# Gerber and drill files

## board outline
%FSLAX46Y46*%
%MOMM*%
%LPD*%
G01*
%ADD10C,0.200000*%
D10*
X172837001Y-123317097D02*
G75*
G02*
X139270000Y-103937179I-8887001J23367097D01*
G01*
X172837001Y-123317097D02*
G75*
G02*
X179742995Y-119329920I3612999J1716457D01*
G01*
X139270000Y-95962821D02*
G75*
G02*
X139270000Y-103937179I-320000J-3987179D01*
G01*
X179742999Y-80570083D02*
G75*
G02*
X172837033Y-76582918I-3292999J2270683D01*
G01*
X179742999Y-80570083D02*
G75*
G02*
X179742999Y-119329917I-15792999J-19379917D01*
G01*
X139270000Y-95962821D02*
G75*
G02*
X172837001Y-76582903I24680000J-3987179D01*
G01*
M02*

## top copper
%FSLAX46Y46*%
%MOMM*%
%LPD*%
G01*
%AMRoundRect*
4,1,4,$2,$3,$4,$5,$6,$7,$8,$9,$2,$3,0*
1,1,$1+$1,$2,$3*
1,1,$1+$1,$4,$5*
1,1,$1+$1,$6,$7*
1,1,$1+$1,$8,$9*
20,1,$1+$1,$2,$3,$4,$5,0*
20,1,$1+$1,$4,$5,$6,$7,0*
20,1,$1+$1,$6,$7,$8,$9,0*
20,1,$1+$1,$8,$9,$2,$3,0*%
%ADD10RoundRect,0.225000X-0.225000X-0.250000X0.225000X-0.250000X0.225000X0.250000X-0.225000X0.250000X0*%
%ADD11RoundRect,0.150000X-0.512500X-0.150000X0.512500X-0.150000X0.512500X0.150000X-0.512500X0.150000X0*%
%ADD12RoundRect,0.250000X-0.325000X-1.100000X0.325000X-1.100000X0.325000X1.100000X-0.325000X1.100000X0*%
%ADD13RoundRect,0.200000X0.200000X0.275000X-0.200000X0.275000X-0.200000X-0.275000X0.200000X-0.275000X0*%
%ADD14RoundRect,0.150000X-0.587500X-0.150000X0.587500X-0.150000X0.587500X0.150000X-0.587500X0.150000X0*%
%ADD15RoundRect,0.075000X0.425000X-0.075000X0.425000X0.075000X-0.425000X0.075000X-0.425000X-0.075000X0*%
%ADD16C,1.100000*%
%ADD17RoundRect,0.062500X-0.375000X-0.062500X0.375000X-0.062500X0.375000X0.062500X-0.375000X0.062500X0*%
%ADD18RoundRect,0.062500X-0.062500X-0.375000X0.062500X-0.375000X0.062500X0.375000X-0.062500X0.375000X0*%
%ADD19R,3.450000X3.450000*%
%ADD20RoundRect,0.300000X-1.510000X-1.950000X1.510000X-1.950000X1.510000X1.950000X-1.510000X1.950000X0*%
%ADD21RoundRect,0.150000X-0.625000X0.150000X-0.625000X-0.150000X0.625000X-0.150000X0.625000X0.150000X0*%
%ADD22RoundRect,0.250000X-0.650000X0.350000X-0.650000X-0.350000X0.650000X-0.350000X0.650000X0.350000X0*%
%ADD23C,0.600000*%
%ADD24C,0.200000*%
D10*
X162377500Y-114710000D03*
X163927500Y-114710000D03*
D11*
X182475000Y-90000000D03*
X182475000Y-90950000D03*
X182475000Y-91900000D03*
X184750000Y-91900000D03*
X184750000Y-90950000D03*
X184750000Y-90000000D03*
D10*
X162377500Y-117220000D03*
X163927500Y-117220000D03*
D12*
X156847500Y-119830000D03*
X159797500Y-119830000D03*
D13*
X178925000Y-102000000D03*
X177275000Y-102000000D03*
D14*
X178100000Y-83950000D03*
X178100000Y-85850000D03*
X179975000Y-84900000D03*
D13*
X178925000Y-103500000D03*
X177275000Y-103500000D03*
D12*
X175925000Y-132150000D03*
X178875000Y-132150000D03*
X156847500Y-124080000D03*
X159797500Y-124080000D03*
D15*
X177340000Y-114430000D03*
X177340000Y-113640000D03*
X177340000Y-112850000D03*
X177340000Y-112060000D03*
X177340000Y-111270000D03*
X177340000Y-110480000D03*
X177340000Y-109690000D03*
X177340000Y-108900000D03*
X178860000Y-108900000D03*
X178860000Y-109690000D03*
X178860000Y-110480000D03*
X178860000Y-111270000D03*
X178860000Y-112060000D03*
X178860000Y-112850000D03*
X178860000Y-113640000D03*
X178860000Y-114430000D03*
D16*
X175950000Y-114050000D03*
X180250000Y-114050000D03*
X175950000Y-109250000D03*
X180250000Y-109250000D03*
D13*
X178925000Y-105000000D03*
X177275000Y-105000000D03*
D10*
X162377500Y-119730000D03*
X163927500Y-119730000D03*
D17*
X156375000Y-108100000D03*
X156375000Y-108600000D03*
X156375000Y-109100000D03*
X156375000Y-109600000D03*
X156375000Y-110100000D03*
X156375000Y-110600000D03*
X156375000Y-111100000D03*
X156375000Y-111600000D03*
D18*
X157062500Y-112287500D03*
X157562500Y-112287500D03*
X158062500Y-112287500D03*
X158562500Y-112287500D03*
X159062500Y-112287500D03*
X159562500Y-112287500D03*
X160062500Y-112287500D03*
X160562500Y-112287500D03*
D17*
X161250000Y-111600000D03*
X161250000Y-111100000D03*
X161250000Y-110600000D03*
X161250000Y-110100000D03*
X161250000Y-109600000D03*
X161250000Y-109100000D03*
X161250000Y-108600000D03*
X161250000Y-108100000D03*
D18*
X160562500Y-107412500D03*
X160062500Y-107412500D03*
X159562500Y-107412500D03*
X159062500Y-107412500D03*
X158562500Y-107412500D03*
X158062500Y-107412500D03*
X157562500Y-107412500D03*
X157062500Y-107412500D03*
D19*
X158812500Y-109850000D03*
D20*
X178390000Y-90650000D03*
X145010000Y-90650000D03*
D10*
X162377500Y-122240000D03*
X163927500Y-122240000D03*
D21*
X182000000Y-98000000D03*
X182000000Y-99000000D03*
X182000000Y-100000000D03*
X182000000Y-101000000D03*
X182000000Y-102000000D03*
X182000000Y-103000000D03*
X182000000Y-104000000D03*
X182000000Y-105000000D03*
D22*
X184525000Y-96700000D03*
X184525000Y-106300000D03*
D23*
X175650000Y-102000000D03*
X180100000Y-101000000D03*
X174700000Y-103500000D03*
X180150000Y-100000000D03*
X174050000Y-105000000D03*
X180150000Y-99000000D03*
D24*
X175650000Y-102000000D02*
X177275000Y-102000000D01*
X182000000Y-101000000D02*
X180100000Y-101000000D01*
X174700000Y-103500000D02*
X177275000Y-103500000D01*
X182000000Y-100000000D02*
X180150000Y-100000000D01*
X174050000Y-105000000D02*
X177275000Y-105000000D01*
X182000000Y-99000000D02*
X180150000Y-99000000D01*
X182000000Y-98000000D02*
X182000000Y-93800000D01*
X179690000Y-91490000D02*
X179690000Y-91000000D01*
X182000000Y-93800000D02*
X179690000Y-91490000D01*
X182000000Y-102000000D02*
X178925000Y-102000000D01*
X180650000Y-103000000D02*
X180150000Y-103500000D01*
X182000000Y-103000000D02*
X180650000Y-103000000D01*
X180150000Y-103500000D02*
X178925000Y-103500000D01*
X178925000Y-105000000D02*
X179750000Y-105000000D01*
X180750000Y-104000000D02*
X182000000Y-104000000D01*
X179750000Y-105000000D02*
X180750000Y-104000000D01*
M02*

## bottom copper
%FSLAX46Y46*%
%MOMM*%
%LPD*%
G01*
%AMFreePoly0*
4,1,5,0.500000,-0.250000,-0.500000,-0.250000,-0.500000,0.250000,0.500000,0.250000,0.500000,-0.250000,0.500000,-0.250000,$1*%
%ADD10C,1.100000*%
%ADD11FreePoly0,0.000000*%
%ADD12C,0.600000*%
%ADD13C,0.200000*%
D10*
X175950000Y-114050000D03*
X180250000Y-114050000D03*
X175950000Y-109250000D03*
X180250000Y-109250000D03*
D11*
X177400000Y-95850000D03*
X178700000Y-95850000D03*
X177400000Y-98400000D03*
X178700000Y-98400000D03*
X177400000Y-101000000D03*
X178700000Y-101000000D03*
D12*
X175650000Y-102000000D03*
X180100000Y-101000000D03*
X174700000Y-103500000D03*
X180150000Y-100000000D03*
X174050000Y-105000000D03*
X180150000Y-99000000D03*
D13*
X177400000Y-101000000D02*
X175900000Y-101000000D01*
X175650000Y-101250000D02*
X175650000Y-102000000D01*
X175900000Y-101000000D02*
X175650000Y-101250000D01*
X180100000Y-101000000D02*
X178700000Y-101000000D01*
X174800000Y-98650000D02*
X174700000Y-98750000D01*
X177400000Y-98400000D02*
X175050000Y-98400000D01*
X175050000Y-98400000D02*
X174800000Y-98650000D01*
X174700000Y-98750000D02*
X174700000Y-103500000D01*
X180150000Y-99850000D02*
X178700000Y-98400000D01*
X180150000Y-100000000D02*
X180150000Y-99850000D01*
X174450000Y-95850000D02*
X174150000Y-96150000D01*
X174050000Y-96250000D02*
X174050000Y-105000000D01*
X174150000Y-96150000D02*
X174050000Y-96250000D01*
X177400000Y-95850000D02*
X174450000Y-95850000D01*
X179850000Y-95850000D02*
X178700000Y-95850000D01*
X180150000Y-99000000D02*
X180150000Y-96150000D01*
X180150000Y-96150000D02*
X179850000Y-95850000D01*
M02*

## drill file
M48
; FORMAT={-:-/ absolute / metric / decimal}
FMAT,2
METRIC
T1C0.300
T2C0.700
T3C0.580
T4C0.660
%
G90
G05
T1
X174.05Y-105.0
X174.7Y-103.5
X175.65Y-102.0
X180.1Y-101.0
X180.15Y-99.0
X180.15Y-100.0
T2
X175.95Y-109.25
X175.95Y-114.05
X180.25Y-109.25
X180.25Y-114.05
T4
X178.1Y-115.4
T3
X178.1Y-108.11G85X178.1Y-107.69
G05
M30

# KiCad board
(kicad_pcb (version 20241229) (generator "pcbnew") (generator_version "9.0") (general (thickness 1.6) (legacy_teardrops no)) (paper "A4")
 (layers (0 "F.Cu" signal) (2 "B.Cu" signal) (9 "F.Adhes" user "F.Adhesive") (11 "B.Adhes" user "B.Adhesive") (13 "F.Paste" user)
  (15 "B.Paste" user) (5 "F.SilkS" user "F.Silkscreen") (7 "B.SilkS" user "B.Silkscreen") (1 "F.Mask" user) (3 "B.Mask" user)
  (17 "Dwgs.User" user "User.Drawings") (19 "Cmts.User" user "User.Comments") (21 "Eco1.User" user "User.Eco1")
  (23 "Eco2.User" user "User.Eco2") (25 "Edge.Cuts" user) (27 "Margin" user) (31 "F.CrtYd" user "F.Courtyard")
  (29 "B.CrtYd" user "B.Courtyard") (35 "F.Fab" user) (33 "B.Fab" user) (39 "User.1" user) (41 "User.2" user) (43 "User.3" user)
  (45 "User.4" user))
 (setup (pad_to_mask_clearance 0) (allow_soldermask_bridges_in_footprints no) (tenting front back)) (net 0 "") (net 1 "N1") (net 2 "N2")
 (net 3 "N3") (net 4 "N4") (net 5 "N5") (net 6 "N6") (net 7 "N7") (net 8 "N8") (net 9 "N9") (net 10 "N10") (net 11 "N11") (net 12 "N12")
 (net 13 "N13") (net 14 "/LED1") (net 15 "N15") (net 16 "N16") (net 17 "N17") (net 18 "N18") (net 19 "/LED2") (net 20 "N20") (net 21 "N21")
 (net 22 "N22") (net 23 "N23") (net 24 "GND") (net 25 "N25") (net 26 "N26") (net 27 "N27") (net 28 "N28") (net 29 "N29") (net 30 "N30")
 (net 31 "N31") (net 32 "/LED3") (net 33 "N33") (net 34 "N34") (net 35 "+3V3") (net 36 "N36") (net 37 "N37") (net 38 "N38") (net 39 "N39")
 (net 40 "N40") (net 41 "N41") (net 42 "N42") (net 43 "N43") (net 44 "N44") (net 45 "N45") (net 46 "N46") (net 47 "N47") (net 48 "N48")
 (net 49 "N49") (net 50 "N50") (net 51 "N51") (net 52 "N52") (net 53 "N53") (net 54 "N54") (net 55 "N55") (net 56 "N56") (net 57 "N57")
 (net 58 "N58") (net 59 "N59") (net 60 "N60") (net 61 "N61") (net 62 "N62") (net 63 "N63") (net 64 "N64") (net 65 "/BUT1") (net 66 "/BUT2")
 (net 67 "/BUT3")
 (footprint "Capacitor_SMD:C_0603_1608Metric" (layer "F.Cu") (at 163.1525 114.71)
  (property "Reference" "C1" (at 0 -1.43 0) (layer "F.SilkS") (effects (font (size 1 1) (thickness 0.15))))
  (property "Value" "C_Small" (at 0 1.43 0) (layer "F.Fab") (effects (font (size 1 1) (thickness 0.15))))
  (pad "1" smd roundrect (at -0.775 0) (size 0.9 0.95) (layers "F.Cu" "F.Mask" "F.Paste") (roundrect_rratio 0.25) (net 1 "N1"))
  (pad "2" smd roundrect (at 0.775 0) (size 0.9 0.95) (layers "F.Cu" "F.Mask" "F.Paste") (roundrect_rratio 0.25) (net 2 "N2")))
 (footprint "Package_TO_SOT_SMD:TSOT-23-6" (layer "F.Cu") (at 183.6125 90.95)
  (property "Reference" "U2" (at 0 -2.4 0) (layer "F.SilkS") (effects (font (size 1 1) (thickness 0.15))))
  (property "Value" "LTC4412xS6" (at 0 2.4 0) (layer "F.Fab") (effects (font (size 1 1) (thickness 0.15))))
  (pad "1" smd roundrect (at -1.1375 -0.95) (size 1.325 0.6) (layers "F.Cu" "F.Mask" "F.Paste") (roundrect_rratio 0.25) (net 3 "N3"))
  (pad "2" smd roundrect (at -1.1375 0) (size 1.325 0.6) (layers "F.Cu" "F.Mask" "F.Paste") (roundrect_rratio 0.25) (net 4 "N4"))
  (pad "3" smd roundrect (at -1.1375 0.95) (size 1.325 0.6) (layers "F.Cu" "F.Mask" "F.Paste") (roundrect_rratio 0.25) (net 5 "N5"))
  (pad "4" smd roundrect (at 1.1375 0.95) (size 1.325 0.6) (layers "F.Cu" "F.Mask" "F.Paste") (roundrect_rratio 0.25) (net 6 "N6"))
  (pad "5" smd roundrect (at 1.1375 0) (size 1.325 0.6) (layers "F.Cu" "F.Mask" "F.Paste") (roundrect_rratio 0.25) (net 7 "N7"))
  (pad "6" smd roundrect (at 1.1375 -0.95) (size 1.325 0.6) (layers "F.Cu" "F.Mask" "F.Paste") (roundrect_rratio 0.25) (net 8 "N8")))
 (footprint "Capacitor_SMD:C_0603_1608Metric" (layer "F.Cu") (at 163.1525 117.22)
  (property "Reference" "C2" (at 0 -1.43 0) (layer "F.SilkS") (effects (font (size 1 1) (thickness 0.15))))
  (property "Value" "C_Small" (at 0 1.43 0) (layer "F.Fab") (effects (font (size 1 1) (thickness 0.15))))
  (pad "1" smd roundrect (at -0.775 0) (size 0.9 0.95) (layers "F.Cu" "F.Mask" "F.Paste") (roundrect_rratio 0.25) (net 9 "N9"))
  (pad "2" smd roundrect (at 0.775 0) (size 0.9 0.95) (layers "F.Cu" "F.Mask" "F.Paste") (roundrect_rratio 0.25) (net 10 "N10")))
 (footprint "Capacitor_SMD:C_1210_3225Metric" (layer "F.Cu") (at 158.3225 119.83)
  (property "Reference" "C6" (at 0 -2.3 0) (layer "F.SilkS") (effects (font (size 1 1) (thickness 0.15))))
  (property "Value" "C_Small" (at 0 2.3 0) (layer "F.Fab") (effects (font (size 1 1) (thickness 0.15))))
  (pad "1" smd roundrect (at -1.475 0) (size 1.15 2.7) (layers "F.Cu" "F.Mask" "F.Paste") (roundrect_rratio 0.217391) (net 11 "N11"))
  (pad "2" smd roundrect (at 1.475 0) (size 1.15 2.7) (layers "F.Cu" "F.Mask" "F.Paste") (roundrect_rratio 0.217391) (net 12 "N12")))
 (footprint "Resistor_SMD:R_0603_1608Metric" (layer "F.Cu") (at 178.1 102 180)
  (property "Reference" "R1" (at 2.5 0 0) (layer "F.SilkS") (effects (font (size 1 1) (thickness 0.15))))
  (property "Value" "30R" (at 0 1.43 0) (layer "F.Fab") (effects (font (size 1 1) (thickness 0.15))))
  (pad "1" smd roundrect (at -0.825 0 180) (size 0.8 0.95) (layers "F.Cu" "F.Mask" "F.Paste") (roundrect_rratio 0.25) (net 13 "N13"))
  (pad "2" smd roundrect (at 0.825 0 180) (size 0.8 0.95) (layers "F.Cu" "F.Mask" "F.Paste") (roundrect_rratio 0.25) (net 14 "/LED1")))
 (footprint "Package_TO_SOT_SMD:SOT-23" (layer "F.Cu") (at 179.0375 84.9)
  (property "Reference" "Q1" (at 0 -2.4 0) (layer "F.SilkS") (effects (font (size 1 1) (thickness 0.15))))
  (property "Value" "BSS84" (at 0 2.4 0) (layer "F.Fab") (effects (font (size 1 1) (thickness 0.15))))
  (pad "1" smd roundrect (at -0.9375 -0.95) (size 1.475 0.6) (layers "F.Cu" "F.Mask" "F.Paste") (roundrect_rratio 0.25) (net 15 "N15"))
  (pad "2" smd roundrect (at -0.9375 0.95) (size 1.475 0.6) (layers "F.Cu" "F.Mask" "F.Paste") (roundrect_rratio 0.25) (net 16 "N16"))
  (pad "3" smd roundrect (at 0.9375 0) (size 1.475 0.6) (layers "F.Cu" "F.Mask" "F.Paste") (roundrect_rratio 0.25) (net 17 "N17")))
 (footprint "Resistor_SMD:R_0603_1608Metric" (layer "F.Cu") (at 178.1 103.5 180)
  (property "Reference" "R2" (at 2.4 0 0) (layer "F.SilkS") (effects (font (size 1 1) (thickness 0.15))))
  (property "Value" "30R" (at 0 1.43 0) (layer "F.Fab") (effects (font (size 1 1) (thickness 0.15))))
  (pad "1" smd roundrect (at -0.825 0 180) (size 0.8 0.95) (layers "F.Cu" "F.Mask" "F.Paste") (roundrect_rratio 0.25) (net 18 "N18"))
  (pad "2" smd roundrect (at 0.825 0 180) (size 0.8 0.95) (layers "F.Cu" "F.Mask" "F.Paste") (roundrect_rratio 0.25) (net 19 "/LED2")))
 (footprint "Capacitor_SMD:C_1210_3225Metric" (layer "F.Cu") (at 177.4 132.15)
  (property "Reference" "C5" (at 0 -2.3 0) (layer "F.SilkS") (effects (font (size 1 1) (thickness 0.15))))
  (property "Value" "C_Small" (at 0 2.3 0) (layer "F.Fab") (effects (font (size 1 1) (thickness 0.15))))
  (pad "1" smd roundrect (at -1.475 0) (size 1.15 2.7) (layers "F.Cu" "F.Mask" "F.Paste") (roundrect_rratio 0.217391) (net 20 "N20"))
  (pad "2" smd roundrect (at 1.475 0) (size 1.15 2.7) (layers "F.Cu" "F.Mask" "F.Paste") (roundrect_rratio 0.217391) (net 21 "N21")))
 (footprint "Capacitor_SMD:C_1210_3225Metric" (layer "F.Cu") (at 158.3225 124.08)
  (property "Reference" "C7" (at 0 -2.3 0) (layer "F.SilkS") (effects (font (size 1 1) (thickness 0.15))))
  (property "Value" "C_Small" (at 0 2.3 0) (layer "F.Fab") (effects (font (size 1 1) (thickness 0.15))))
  (pad "1" smd roundrect (at -1.475 0) (size 1.15 2.7) (layers "F.Cu" "F.Mask" "F.Paste") (roundrect_rratio 0.217391) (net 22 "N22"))
  (pad "2" smd roundrect (at 1.475 0) (size 1.15 2.7) (layers "F.Cu" "F.Mask" "F.Paste") (roundrect_rratio 0.217391) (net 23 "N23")))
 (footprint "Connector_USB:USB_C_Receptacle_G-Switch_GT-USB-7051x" (layer "F.Cu") (at 178.1 111.65 90)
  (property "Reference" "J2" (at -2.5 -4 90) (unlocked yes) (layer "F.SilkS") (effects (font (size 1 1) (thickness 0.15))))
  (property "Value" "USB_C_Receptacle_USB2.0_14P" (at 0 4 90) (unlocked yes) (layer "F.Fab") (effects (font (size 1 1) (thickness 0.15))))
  (pad "" np_thru_hole circle (at -3.75 0 90) (size 0.66 0.66) (drill 0.66) (layers "*.Cu" "*.Mask"))
  (pad "" np_thru_hole oval (at 3.75 0 90) (size 1 0.58) (drill oval 1 0.58) (layers "*.Cu" "*.Mask"))
  (pad "A1" smd roundrect (at -2.78 -0.76 90) (size 0.3 1) (layers "F.Cu" "F.Mask" "F.Paste") (roundrect_rratio 0.25) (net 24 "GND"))
  (pad "A4" smd roundrect (at -1.99 -0.76 90) (size 0.3 1) (layers "F.Cu" "F.Mask" "F.Paste") (roundrect_rratio 0.25) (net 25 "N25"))
  (pad "A5" smd roundrect (at -1.2 -0.76 90) (size 0.3 1) (layers "F.Cu" "F.Mask" "F.Paste") (roundrect_rratio 0.25) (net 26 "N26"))
  (pad "A6" smd roundrect (at -0.41 -0.76 90) (size 0.3 1) (layers "F.Cu" "F.Mask" "F.Paste") (roundrect_rratio 0.25) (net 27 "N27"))
  (pad "A7" smd roundrect (at 0.38 -0.76 90) (size 0.3 1) (layers "F.Cu" "F.Mask" "F.Paste") (roundrect_rratio 0.25) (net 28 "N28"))
  (pad "A8" smd roundrect (at 1.17 -0.76 90) (size 0.3 1) (layers "F.Cu" "F.Mask" "F.Paste") (roundrect_rratio 0.25))
  (pad "A9" smd roundrect (at 1.96 -0.76 90) (size 0.3 1) (layers "F.Cu" "F.Mask" "F.Paste") (roundrect_rratio 0.25) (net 25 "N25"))
  (pad "A12" smd roundrect (at 2.75 -0.76 90) (size 0.3 1) (layers "F.Cu" "F.Mask" "F.Paste") (roundrect_rratio 0.25) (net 24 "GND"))
  (pad "B1" smd roundrect (at 2.75 0.76 90) (size 0.3 1) (layers "F.Cu" "F.Mask" "F.Paste") (roundrect_rratio 0.25) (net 24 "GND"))
  (pad "B4" smd roundrect (at 1.96 0.76 90) (size 0.3 1) (layers "F.Cu" "F.Mask" "F.Paste") (roundrect_rratio 0.25) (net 25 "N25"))
  (pad "B5" smd roundrect (at 1.17 0.76 90) (size 0.3 1) (layers "F.Cu" "F.Mask" "F.Paste") (roundrect_rratio 0.25) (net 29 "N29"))
  (pad "B6" smd roundrect (at 0.38 0.76 90) (size 0.3 1) (layers "F.Cu" "F.Mask" "F.Paste") (roundrect_rratio 0.25) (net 27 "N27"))
  (pad "B7" smd roundrect (at -0.41 0.76 90) (size 0.3 1) (layers "F.Cu" "F.Mask" "F.Paste") (roundrect_rratio 0.25) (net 28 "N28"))
  (pad "B8" smd roundrect (at -1.2 0.76 90) (size 0.3 1) (layers "F.Cu" "F.Mask" "F.Paste") (roundrect_rratio 0.25))
  (pad "B9" smd roundrect (at -1.99 0.76 90) (size 0.3 1) (layers "F.Cu" "F.Mask" "F.Paste") (roundrect_rratio 0.25) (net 25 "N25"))
  (pad "B12" smd roundrect (at -2.78 0.76 90) (size 0.3 1) (layers "F.Cu" "F.Mask" "F.Paste") (roundrect_rratio 0.25) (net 24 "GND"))
  (pad "S1" thru_hole circle (at -2.4 -2.15 90) (size 1.1 1.1) (drill 0.7) (layers "*.Cu" "*.Mask" "F.Paste") (remove_unused_layers no)
   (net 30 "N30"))
  (pad "S1" thru_hole circle (at -2.4 2.15 90) (size 1.1 1.1) (drill 0.7) (layers "*.Cu" "*.Mask" "F.Paste") (remove_unused_layers no)
   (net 30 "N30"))
  (pad "S1" thru_hole circle (at 2.4 -2.15 90) (size 1.1 1.1) (drill 0.7) (layers "*.Cu" "*.Mask" "F.Paste") (remove_unused_layers no)
   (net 30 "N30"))
  (pad "S1" thru_hole circle (at 2.4 2.15 90) (size 1.1 1.1) (drill 0.7) (layers "*.Cu" "*.Mask" "F.Paste") (remove_unused_layers no)
   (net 30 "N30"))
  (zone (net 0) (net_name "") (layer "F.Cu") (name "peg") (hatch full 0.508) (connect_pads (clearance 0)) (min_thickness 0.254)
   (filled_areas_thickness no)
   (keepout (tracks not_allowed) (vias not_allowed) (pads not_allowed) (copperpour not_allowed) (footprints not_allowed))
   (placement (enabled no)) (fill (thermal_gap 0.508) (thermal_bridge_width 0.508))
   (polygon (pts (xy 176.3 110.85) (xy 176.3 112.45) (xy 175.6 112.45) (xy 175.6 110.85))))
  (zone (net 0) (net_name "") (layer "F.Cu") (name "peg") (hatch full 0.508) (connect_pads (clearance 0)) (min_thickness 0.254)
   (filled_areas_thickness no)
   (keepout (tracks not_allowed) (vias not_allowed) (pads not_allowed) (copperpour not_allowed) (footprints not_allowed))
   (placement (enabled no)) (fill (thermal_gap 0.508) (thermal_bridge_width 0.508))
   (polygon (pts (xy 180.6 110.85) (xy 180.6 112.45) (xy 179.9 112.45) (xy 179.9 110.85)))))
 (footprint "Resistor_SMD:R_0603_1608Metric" (layer "F.Cu") (at 178.1 105 180)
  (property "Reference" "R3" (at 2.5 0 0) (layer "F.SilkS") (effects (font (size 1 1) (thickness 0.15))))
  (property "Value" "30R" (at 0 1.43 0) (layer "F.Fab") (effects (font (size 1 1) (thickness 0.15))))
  (pad "1" smd roundrect (at -0.825 0 180) (size 0.8 0.95) (layers "F.Cu" "F.Mask" "F.Paste") (roundrect_rratio 0.25) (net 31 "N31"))
  (pad "2" smd roundrect (at 0.825 0 180) (size 0.8 0.95) (layers "F.Cu" "F.Mask" "F.Paste") (roundrect_rratio 0.25) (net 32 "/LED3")))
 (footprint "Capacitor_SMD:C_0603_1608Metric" (layer "F.Cu") (at 163.1525 119.73)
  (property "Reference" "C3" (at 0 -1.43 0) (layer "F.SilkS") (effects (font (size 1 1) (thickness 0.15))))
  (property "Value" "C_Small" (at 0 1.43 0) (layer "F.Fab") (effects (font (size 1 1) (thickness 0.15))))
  (pad "1" smd roundrect (at -0.775 0) (size 0.9 0.95) (layers "F.Cu" "F.Mask" "F.Paste") (roundrect_rratio 0.25) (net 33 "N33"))
  (pad "2" smd roundrect (at 0.775 0) (size 0.9 0.95) (layers "F.Cu" "F.Mask" "F.Paste") (roundrect_rratio 0.25) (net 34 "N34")))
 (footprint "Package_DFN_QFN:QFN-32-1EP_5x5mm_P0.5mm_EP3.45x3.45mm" (layer "F.Cu") (at 158.8125 109.85)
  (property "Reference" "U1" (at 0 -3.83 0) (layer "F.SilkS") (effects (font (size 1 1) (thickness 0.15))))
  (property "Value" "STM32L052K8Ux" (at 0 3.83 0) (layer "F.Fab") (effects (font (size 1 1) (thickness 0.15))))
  (pad "" smd roundrect (at -1.15 -1.15) (size 0.93 0.93) (layers "F.Paste") (roundrect_rratio 0.25))
  (pad "" smd roundrect (at -1.15 0) (size 0.93 0.93) (layers "F.Paste") (roundrect_rratio 0.25))
  (pad "" smd roundrect (at -1.15 1.15) (size 0.93 0.93) (layers "F.Paste") (roundrect_rratio 0.25))
  (pad "" smd roundrect (at 0 -1.15) (size 0.93 0.93) (layers "F.Paste") (roundrect_rratio 0.25))
  (pad "" smd roundrect (at 0 0) (size 0.93 0.93) (layers "F.Paste") (roundrect_rratio 0.25))
  (pad "" smd roundrect (at 0 1.15) (size 0.93 0.93) (layers "F.Paste") (roundrect_rratio 0.25))
  (pad "" smd roundrect (at 1.15 -1.15) (size 0.93 0.93) (layers "F.Paste") (roundrect_rratio 0.25))
  (pad "" smd roundrect (at 1.15 0) (size 0.93 0.93) (layers "F.Paste") (roundrect_rratio 0.25))
  (pad "" smd roundrect (at 1.15 1.15) (size 0.93 0.93) (layers "F.Paste") (roundrect_rratio 0.25))
  (pad "1" smd roundrect (at -2.4375 -1.75) (size 0.875 0.25) (layers "F.Cu" "F.Mask" "F.Paste") (roundrect_rratio 0.25) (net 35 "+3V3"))
  (pad "2" smd roundrect (at -2.4375 -1.25) (size 0.875 0.25) (layers "F.Cu" "F.Mask" "F.Paste") (roundrect_rratio 0.25) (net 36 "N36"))
  (pad "3" smd roundrect (at -2.4375 -0.75) (size 0.875 0.25) (layers "F.Cu" "F.Mask" "F.Paste") (roundrect_rratio 0.25) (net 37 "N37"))
  (pad "4" smd roundrect (at -2.4375 -0.25) (size 0.875 0.25) (layers "F.Cu" "F.Mask" "F.Paste") (roundrect_rratio 0.25) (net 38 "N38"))
  (pad "5" smd roundrect (at -2.4375 0.25) (size 0.875 0.25) (layers "F.Cu" "F.Mask" "F.Paste") (roundrect_rratio 0.25) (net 35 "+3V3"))
  (pad "6" smd roundrect (at -2.4375 0.75) (size 0.875 0.25) (layers "F.Cu" "F.Mask" "F.Paste") (roundrect_rratio 0.25) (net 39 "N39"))
  (pad "7" smd roundrect (at -2.4375 1.25) (size 0.875 0.25) (layers "F.Cu" "F.Mask" "F.Paste") (roundrect_rratio 0.25) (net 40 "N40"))
  (pad "8" smd roundrect (at -2.4375 1.75) (size 0.875 0.25) (layers "F.Cu" "F.Mask" "F.Paste") (roundrect_rratio 0.25) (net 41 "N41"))
  (pad "9" smd roundrect (at -1.75 2.4375) (size 0.25 0.875) (layers "F.Cu" "F.Mask" "F.Paste") (roundrect_rratio 0.25) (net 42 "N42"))
  (pad "10" smd roundrect (at -1.25 2.4375) (size 0.25 0.875) (layers "F.Cu" "F.Mask" "F.Paste") (roundrect_rratio 0.25) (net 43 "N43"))
  (pad "11" smd roundrect (at -0.75 2.4375) (size 0.25 0.875) (layers "F.Cu" "F.Mask" "F.Paste") (roundrect_rratio 0.25) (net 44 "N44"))
  (pad "12" smd roundrect (at -0.25 2.4375) (size 0.25 0.875) (layers "F.Cu" "F.Mask" "F.Paste") (roundrect_rratio 0.25) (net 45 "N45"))
  (pad "13" smd roundrect (at 0.25 2.4375) (size 0.25 0.875) (layers "F.Cu" "F.Mask" "F.Paste") (roundrect_rratio 0.25) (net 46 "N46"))
  (pad "14" smd roundrect (at 0.75 2.4375) (size 0.25 0.875) (layers "F.Cu" "F.Mask" "F.Paste") (roundrect_rratio 0.25) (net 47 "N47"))
  (pad "15" smd roundrect (at 1.25 2.4375) (size 0.25 0.875) (layers "F.Cu" "F.Mask" "F.Paste") (roundrect_rratio 0.25) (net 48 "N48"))
  (pad "16" smd roundrect (at 1.75 2.4375) (size 0.25 0.875) (layers "F.Cu" "F.Mask" "F.Paste") (roundrect_rratio 0.25) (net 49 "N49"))
  (pad "17" smd roundrect (at 2.4375 1.75) (size 0.875 0.25) (layers "F.Cu" "F.Mask" "F.Paste") (roundrect_rratio 0.25) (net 35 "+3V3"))
  (pad "18" smd roundrect (at 2.4375 1.25) (size 0.875 0.25) (layers "F.Cu" "F.Mask" "F.Paste") (roundrect_rratio 0.25) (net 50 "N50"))
  (pad "19" smd roundrect (at 2.4375 0.75) (size 0.875 0.25) (layers "F.Cu" "F.Mask" "F.Paste") (roundrect_rratio 0.25) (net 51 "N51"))
  (pad "20" smd roundrect (at 2.4375 0.25) (size 0.875 0.25) (layers "F.Cu" "F.Mask" "F.Paste") (roundrect_rratio 0.25) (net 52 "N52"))
  (pad "21" smd roundrect (at 2.4375 -0.25) (size 0.875 0.25) (layers "F.Cu" "F.Mask" "F.Paste") (roundrect_rratio 0.25) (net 28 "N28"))
  (pad "22" smd roundrect (at 2.4375 -0.75) (size 0.875 0.25) (layers "F.Cu" "F.Mask" "F.Paste") (roundrect_rratio 0.25) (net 27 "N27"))
  (pad "23" smd roundrect (at 2.4375 -1.25) (size 0.875 0.25) (layers "F.Cu" "F.Mask" "F.Paste") (roundrect_rratio 0.25) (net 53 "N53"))
  (pad "24" smd roundrect (at 2.4375 -1.75) (size 0.875 0.25) (layers "F.Cu" "F.Mask" "F.Paste") (roundrect_rratio 0.25) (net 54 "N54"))
  (pad "25" smd roundrect (at 1.75 -2.4375) (size 0.25 0.875) (layers "F.Cu" "F.Mask" "F.Paste") (roundrect_rratio 0.25) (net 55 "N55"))
  (pad "26" smd roundrect (at 1.25 -2.4375) (size 0.25 0.875) (layers "F.Cu" "F.Mask" "F.Paste") (roundrect_rratio 0.25) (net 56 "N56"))
  (pad "27" smd roundrect (at 0.75 -2.4375) (size 0.25 0.875) (layers "F.Cu" "F.Mask" "F.Paste") (roundrect_rratio 0.25) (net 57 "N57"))
  (pad "28" smd roundrect (at 0.25 -2.4375) (size 0.25 0.875) (layers "F.Cu" "F.Mask" "F.Paste") (roundrect_rratio 0.25) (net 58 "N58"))
  (pad "29" smd roundrect (at -0.25 -2.4375) (size 0.25 0.875) (layers "F.Cu" "F.Mask" "F.Paste") (roundrect_rratio 0.25) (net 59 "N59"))
  (pad "30" smd roundrect (at -0.75 -2.4375) (size 0.25 0.875) (layers "F.Cu" "F.Mask" "F.Paste") (roundrect_rratio 0.25) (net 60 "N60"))
  (pad "31" smd roundrect (at -1.25 -2.4375) (size 0.25 0.875) (layers "F.Cu" "F.Mask" "F.Paste") (roundrect_rratio 0.25) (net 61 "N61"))
  (pad "32" smd roundrect (at -1.75 -2.4375) (size 0.25 0.875) (layers "F.Cu" "F.Mask" "F.Paste") (roundrect_rratio 0.25) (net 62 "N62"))
  (pad "33" smd rect (at 0 0) (size 3.45 3.45) (layers "F.Cu" "F.Mask") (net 24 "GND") (zone_connect 2)))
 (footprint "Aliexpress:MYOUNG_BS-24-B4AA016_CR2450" (layer "F.Cu") (at 161.7 90.65)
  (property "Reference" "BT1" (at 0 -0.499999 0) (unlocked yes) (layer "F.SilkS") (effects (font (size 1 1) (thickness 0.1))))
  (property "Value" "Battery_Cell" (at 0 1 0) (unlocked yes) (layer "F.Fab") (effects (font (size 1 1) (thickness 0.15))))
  (pad "1" smd roundrect (at 16.69 0) (size 3.62 4.5) (layers "F.Cu" "F.Mask" "F.Paste") (roundrect_rratio 0.08287292818) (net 35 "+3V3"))
  (pad "2" smd roundrect (at -16.69 0) (size 3.62 4.5) (layers "F.Cu" "F.Mask" "F.Paste") (roundrect_rratio 0.08287292818) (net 24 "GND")))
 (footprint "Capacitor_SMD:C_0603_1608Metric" (layer "F.Cu") (at 163.1525 122.24)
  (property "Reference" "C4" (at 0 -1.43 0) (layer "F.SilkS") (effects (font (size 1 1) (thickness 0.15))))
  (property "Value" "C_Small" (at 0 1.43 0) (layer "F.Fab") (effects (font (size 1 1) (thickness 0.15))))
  (pad "1" smd roundrect (at -0.775 0) (size 0.9 0.95) (layers "F.Cu" "F.Mask" "F.Paste") (roundrect_rratio 0.25) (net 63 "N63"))
  (pad "2" smd roundrect (at 0.775 0) (size 0.9 0.95) (layers "F.Cu" "F.Mask" "F.Paste") (roundrect_rratio 0.25) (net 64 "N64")))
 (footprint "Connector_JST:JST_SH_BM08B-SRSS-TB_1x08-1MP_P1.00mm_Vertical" (layer "F.Cu") (at 183.325 101.5 -90)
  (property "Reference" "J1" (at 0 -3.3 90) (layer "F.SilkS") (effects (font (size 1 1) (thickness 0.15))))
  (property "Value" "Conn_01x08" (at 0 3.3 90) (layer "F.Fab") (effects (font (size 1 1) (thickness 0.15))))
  (pad "1" smd roundrect (at -3.5 1.325 270) (size 0.6 1.55) (layers "F.Cu" "F.Mask" "F.Paste") (roundrect_rratio 0.25) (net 35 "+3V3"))
  (pad "2" smd roundrect (at -2.5 1.325 270) (size 0.6 1.55) (layers "F.Cu" "F.Mask" "F.Paste") (roundrect_rratio 0.25) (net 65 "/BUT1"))
  (pad "3" smd roundrect (at -1.5 1.325 270) (size 0.6 1.55) (layers "F.Cu" "F.Mask" "F.Paste") (roundrect_rratio 0.25) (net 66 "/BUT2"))
  (pad "4" smd roundrect (at -0.5 1.325 270) (size 0.6 1.55) (layers "F.Cu" "F.Mask" "F.Paste") (roundrect_rratio 0.25) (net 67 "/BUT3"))
  (pad "5" smd roundrect (at 0.5 1.325 270) (size 0.6 1.55) (layers "F.Cu" "F.Mask" "F.Paste") (roundrect_rratio 0.25) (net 13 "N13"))
  (pad "6" smd roundrect (at 1.5 1.325 270) (size 0.6 1.55) (layers "F.Cu" "F.Mask" "F.Paste") (roundrect_rratio 0.25) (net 18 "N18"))
  (pad "7" smd roundrect (at 2.5 1.325 270) (size 0.6 1.55) (layers "F.Cu" "F.Mask" "F.Paste") (roundrect_rratio 0.25) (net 31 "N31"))
  (pad "8" smd roundrect (at 3.5 1.325 270) (size 0.6 1.55) (layers "F.Cu" "F.Mask" "F.Paste") (roundrect_rratio 0.25) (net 24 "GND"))
  (pad "MP" smd roundrect (at -4.8 -1.2 270) (size 1.2 1.8) (layers "F.Cu" "F.Mask" "F.Paste") (roundrect_rratio 0.208333))
  (pad "MP" smd roundrect (at 4.8 -1.2 270) (size 1.2 1.8) (layers "F.Cu" "F.Mask" "F.Paste") (roundrect_rratio 0.208333)))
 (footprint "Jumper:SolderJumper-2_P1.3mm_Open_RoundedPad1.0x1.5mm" (layer "B.Cu") (at 178.05 95.85)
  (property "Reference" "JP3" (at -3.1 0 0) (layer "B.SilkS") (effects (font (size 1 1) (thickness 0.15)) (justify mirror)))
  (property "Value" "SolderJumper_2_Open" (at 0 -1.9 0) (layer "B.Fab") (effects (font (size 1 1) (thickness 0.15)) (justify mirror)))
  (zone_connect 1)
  (pad "1" smd custom (at -0.65 0) (size 1 0.5) (layers "B.Cu" "B.Mask") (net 32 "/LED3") (zone_connect 2) (thermal_bridge_angle 45)
   (options (clearance outline) (anchor rect)) (primitives))
  (pad "2" smd custom (at 0.65 0) (size 1 0.5) (layers "B.Cu" "B.Mask") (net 65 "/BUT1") (zone_connect 2) (thermal_bridge_angle 45)
   (options (clearance outline) (anchor rect)) (primitives)))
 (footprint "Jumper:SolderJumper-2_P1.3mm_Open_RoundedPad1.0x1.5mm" (layer "B.Cu") (at 178.05 98.4)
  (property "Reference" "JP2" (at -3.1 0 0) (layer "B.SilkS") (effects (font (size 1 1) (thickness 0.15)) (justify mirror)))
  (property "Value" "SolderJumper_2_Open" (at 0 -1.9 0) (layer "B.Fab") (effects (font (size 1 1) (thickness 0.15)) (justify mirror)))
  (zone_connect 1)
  (pad "1" smd custom (at -0.65 0) (size 1 0.5) (layers "B.Cu" "B.Mask") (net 19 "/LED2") (zone_connect 2) (thermal_bridge_angle 45)
   (options (clearance outline) (anchor rect)) (primitives))
  (pad "2" smd custom (at 0.65 0) (size 1 0.5) (layers "B.Cu" "B.Mask") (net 66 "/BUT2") (zone_connect 2) (thermal_bridge_angle 45)
   (options (clearance outline) (anchor rect)) (primitives)))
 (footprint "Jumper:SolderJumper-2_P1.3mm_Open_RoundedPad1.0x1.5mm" (layer "B.Cu") (at 178.05 101)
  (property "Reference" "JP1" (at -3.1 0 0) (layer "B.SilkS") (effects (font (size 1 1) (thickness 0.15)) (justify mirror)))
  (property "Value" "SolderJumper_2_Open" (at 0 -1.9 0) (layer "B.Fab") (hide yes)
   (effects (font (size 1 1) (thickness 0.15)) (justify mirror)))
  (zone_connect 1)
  (pad "1" smd custom (at -0.65 0) (size 1 0.5) (layers "B.Cu" "B.Mask") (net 14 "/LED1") (zone_connect 2) (thermal_bridge_angle 45)
   (options (clearance outline) (anchor rect)) (primitives))
  (pad "2" smd custom (at 0.65 0) (size 1 0.5) (layers "B.Cu" "B.Mask") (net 67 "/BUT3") (zone_connect 2) (thermal_bridge_angle 45)
   (options (clearance outline) (anchor rect)) (primitives)))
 (gr_arc (start 172.837001 123.317097) (mid 151.45 121.600635) (end 139.27 103.937179) (stroke (width 0.2) (type default))
  (layer "Edge.Cuts"))
 (gr_arc (start 172.837001 123.317097) (mid 174.450001 118.13654) (end 179.742999 119.329917) (stroke (width 0.2) (type default))
  (layer "Edge.Cuts"))
 (gr_arc (start 139.27 95.962821) (mid 142.95 99.95) (end 139.27 103.937179) (stroke (width 0.2) (type default)) (layer "Edge.Cuts"))
 (gr_arc (start 179.742999 80.570083) (mid 174.45 81.763467) (end 172.837001 76.582903) (stroke (width 0.2) (type default))
  (layer "Edge.Cuts"))
 (gr_arc (start 179.742999 80.570083) (mid 188.95 99.95) (end 179.742999 119.329917) (stroke (width 0.2) (type default)) (layer "Edge.Cuts"))
 (gr_arc (start 139.27 95.962821) (mid 151.45 78.299365) (end 172.837001 76.582903) (stroke (width 0.2) (type default)) (layer "Edge.Cuts"))
 (segment (start 175.65 102) (end 177.275 102) (width 0.2) (layer "F.Cu") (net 14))
 (via (at 175.65 102) (size 0.6) (drill 0.3) (layers "F.Cu" "B.Cu") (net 14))
 (segment (start 177.4 101) (end 175.9 101) (width 0.2) (layer "B.Cu") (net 14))
 (segment (start 175.65 101.25) (end 175.65 102) (width 0.2) (layer "B.Cu") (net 14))
 (segment (start 175.9 101) (end 175.65 101.25) (width 0.2) (layer "B.Cu") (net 14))
 (segment (start 182 101) (end 180.1 101) (width 0.2) (layer "F.Cu") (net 67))
 (via (at 180.1 101) (size 0.6) (drill 0.3) (layers "F.Cu" "B.Cu") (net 67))
 (segment (start 180.1 101) (end 178.7 101) (width 0.2) (layer "B.Cu") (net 67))
 (segment (start 174.7 103.5) (end 177.275 103.5) (width 0.2) (layer "F.Cu") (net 19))
 (via (at 174.7 103.5) (size 0.6) (drill 0.3) (layers "F.Cu" "B.Cu") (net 19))
 (segment (start 174.8 98.65) (end 174.7 98.75) (width 0.2) (layer "B.Cu") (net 19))
 (segment (start 177.4 98.4) (end 175.05 98.4) (width 0.2) (layer "B.Cu") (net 19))
 (segment (start 175.05 98.4) (end 174.8 98.65) (width 0.2) (layer "B.Cu") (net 19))
 (segment (start 174.7 98.75) (end 174.7 103.5) (width 0.2) (layer "B.Cu") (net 19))
 (segment (start 182 100) (end 180.15 100) (width 0.2) (layer "F.Cu") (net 66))
 (via (at 180.15 100) (size 0.6) (drill 0.3) (layers "F.Cu" "B.Cu") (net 66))
 (segment (start 180.15 99.85) (end 178.7 98.4) (width 0.2) (layer "B.Cu") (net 66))
 (segment (start 180.15 100) (end 180.15 99.85) (width 0.2) (layer "B.Cu") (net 66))
 (segment (start 174.05 105) (end 177.275 105) (width 0.2) (layer "F.Cu") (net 32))
 (via (at 174.05 105) (size 0.6) (drill 0.3) (layers "F.Cu" "B.Cu") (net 32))
 (segment (start 174.45 95.85) (end 174.15 96.15) (width 0.2) (layer "B.Cu") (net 32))
 (segment (start 174.05 96.25) (end 174.05 105) (width 0.2) (layer "B.Cu") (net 32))
 (segment (start 174.15 96.15) (end 174.05 96.25) (width 0.2) (layer "B.Cu") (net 32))
 (segment (start 177.4 95.85) (end 174.45 95.85) (width 0.2) (layer "B.Cu") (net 32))
 (segment (start 182 99) (end 180.15 99) (width 0.2) (layer "F.Cu") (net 65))
 (via (at 180.15 99) (size 0.6) (drill 0.3) (layers "F.Cu" "B.Cu") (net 65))
 (segment (start 179.85 95.85) (end 178.7 95.85) (width 0.2) (layer "B.Cu") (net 65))
 (segment (start 180.15 99) (end 180.15 96.15) (width 0.2) (layer "B.Cu") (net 65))
 (segment (start 180.15 96.15) (end 179.85 95.85) (width 0.2) (layer "B.Cu") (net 65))
 (segment (start 182 98) (end 182 93.8) (width 0.2) (layer "F.Cu") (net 35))
 (segment (start 179.69 91.49) (end 179.69 91) (width 0.2) (layer "F.Cu") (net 35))
 (segment (start 182 93.8) (end 179.69 91.49) (width 0.2) (layer "F.Cu") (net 35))
 (segment (start 182 102) (end 178.925 102) (width 0.2) (layer "F.Cu") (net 13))
 (segment (start 180.65 103) (end 180.15 103.5) (width 0.2) (layer "F.Cu") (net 18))
 (segment (start 182 103) (end 180.65 103) (width 0.2) (layer "F.Cu") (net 18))
 (segment (start 180.15 103.5) (end 178.925 103.5) (width 0.2) (layer "F.Cu") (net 18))
 (segment (start 178.925 105) (end 179.75 105) (width 0.2) (layer "F.Cu") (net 31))
 (segment (start 180.75 104) (end 182 104) (width 0.2) (layer "F.Cu") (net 31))
 (segment (start 179.75 105) (end 180.75 104) (width 0.2) (layer "F.Cu") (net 31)))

